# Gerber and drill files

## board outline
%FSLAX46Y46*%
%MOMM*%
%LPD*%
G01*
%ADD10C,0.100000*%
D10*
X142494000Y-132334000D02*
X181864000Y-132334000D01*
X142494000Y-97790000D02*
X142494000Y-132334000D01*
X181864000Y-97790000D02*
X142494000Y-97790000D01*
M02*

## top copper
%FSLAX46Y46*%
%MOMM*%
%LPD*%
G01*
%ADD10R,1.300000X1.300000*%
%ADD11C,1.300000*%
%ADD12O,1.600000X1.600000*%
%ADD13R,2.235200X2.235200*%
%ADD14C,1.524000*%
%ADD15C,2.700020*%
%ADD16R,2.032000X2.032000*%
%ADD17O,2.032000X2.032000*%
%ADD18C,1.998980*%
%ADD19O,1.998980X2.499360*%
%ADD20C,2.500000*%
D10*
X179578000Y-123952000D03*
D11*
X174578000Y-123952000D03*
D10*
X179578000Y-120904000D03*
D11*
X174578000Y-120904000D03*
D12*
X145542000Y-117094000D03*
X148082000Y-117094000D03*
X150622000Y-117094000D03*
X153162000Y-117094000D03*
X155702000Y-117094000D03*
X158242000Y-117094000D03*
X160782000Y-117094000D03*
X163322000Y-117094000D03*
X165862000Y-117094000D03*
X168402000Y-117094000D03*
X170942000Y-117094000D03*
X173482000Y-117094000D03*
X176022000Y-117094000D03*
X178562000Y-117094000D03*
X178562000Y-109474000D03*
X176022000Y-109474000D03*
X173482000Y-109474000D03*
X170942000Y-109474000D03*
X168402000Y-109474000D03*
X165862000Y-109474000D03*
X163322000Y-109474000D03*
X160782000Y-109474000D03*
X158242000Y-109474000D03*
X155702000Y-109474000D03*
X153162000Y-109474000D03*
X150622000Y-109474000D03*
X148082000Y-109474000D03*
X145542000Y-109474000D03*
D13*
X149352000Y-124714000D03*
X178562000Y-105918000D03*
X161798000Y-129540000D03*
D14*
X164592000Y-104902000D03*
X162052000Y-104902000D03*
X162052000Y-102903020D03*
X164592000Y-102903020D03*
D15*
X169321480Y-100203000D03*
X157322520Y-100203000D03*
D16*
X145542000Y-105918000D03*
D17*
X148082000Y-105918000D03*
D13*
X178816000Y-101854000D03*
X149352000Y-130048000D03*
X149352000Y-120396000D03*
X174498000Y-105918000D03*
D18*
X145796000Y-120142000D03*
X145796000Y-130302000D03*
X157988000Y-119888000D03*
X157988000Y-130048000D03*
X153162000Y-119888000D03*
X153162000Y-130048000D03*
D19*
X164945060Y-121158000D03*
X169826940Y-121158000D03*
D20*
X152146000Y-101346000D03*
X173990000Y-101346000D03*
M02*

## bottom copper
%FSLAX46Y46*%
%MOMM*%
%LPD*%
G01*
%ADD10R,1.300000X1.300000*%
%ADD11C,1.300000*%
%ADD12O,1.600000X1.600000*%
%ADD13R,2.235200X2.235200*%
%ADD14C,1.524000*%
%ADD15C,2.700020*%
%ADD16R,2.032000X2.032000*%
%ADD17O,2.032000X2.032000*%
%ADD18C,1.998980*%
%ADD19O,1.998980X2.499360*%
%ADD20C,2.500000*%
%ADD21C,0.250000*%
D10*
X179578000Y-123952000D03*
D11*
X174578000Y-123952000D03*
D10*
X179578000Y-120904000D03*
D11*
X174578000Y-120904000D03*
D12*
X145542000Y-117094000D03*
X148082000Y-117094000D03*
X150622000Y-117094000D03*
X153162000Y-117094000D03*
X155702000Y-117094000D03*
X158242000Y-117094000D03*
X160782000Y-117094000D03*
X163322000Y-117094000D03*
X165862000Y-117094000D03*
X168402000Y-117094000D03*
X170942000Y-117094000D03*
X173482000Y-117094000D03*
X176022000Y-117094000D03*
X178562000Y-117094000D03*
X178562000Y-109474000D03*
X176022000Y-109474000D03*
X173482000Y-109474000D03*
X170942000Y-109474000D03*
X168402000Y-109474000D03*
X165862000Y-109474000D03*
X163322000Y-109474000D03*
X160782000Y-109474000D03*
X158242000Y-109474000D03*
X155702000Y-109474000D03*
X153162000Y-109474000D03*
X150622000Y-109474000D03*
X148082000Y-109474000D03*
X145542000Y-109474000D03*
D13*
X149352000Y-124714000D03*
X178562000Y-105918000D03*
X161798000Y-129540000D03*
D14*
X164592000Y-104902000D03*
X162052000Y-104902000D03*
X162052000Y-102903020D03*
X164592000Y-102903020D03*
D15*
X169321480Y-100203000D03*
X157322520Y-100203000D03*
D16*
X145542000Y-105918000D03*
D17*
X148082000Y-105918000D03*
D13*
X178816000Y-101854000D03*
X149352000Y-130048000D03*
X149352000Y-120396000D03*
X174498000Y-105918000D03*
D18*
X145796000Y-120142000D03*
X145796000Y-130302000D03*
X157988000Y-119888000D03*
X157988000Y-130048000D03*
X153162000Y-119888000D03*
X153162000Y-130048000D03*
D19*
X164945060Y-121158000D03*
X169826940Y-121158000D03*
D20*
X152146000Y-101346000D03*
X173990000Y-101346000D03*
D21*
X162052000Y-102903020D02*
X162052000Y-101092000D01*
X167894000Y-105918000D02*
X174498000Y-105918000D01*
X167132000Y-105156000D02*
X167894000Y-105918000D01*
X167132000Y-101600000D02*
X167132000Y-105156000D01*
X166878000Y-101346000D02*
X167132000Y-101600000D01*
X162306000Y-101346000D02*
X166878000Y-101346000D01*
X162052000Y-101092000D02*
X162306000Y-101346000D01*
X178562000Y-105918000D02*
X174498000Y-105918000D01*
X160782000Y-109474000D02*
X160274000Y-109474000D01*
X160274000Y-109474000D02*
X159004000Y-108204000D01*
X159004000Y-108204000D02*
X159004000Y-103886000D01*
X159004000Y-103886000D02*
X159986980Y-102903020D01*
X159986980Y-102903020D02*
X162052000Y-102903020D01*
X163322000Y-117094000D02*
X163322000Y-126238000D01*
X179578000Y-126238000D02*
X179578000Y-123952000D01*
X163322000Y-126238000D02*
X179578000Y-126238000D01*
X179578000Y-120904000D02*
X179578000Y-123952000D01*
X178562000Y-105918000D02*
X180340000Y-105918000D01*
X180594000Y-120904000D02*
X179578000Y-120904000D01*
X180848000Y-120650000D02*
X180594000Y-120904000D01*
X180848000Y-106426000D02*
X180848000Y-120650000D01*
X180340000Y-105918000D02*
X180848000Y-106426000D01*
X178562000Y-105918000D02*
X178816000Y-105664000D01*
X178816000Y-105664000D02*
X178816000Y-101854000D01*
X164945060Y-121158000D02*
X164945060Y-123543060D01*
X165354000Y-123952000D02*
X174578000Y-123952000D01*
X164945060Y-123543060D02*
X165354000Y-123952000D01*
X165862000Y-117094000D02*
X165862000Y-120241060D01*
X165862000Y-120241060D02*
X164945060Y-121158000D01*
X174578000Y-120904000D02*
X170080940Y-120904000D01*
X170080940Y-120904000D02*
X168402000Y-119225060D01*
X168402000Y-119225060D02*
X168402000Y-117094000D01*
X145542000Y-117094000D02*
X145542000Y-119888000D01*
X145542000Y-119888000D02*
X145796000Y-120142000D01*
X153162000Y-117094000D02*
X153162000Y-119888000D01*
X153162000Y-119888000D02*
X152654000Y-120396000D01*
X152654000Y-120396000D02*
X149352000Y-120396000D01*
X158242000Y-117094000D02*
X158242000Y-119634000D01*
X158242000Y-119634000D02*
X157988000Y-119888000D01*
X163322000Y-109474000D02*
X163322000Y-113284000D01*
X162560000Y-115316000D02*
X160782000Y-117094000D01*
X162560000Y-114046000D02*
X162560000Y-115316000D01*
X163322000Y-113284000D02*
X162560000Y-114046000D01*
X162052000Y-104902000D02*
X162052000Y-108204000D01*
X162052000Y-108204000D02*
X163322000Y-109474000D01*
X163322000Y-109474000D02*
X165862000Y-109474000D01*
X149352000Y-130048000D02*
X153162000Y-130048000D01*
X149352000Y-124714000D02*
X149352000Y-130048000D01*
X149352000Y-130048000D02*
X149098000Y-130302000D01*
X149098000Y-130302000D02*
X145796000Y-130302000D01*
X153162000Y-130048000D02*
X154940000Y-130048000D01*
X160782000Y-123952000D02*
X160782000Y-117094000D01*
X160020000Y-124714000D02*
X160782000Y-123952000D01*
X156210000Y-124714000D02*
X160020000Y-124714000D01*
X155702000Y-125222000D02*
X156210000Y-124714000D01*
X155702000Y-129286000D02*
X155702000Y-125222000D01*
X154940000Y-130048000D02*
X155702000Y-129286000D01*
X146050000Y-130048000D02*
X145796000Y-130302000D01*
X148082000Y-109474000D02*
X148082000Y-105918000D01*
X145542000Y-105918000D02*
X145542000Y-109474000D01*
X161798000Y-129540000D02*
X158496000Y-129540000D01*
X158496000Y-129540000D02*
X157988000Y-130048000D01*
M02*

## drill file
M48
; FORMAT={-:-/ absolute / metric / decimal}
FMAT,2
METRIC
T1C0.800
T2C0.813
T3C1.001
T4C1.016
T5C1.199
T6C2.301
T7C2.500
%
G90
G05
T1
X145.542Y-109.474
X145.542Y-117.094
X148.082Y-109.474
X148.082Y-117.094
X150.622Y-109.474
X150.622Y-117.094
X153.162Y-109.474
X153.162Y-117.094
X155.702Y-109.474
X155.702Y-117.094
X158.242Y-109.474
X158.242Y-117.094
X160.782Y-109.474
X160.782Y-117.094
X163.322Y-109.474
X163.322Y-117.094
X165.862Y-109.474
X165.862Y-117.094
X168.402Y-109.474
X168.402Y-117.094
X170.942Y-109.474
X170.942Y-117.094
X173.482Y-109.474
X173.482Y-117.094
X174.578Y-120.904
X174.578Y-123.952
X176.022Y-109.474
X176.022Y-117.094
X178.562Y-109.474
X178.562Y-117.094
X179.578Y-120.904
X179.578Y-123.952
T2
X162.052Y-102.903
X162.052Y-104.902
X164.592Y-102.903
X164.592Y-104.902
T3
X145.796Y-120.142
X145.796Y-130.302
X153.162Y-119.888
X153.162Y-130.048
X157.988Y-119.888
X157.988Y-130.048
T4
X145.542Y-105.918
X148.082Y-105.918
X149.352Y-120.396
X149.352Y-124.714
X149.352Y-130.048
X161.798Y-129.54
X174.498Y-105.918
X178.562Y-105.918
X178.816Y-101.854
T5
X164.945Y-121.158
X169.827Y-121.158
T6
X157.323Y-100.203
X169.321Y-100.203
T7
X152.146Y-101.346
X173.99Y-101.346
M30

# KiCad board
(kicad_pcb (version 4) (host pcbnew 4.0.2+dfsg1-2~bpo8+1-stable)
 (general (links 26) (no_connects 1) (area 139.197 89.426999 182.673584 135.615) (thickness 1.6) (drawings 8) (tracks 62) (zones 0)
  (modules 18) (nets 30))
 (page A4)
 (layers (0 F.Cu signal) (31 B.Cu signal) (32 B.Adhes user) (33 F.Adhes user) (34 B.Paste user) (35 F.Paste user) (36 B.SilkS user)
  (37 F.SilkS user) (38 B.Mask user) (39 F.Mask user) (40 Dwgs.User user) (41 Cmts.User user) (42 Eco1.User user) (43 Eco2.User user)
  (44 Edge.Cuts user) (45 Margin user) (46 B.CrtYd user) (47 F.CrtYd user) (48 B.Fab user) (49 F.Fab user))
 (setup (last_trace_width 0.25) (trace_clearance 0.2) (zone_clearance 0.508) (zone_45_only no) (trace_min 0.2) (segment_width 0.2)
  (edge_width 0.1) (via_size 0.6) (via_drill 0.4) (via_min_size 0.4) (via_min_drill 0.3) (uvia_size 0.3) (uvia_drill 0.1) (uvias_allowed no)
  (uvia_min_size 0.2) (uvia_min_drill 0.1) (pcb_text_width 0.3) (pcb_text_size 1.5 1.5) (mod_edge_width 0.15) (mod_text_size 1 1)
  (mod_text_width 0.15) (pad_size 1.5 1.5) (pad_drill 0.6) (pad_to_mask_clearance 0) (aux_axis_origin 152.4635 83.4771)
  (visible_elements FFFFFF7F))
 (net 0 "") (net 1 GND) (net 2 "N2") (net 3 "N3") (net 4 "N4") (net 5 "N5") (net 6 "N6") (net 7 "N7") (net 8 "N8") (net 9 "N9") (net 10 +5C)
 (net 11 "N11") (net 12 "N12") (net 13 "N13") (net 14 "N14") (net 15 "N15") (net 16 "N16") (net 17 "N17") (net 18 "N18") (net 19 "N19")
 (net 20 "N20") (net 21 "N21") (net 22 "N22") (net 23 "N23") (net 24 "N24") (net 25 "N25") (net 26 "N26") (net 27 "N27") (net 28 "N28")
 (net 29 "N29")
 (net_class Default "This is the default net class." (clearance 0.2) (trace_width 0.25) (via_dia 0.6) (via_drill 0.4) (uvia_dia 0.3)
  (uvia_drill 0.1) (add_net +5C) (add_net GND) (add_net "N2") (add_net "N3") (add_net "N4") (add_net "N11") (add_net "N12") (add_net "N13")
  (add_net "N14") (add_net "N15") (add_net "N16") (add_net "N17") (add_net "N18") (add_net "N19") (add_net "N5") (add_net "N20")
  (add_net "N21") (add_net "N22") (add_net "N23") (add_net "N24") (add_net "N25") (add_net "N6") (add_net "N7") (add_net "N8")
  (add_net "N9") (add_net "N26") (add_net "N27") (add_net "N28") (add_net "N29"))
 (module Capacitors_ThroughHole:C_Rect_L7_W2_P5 (layer F.Cu) (at 179.578 123.952 180)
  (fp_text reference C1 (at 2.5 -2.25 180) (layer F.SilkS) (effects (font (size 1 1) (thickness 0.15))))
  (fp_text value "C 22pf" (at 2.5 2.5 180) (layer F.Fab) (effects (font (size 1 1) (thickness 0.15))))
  (pad 1 thru_hole rect (at 0 0 180) (size 1.3 1.3) (drill 0.8) (layers *.Cu *.Mask F.SilkS) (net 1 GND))
  (pad 2 thru_hole circle (at 5 0 180) (size 1.3 1.3) (drill 0.8) (layers *.Cu *.Mask F.SilkS) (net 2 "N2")))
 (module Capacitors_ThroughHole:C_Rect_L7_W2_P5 (layer F.Cu) (at 179.578 120.904 180)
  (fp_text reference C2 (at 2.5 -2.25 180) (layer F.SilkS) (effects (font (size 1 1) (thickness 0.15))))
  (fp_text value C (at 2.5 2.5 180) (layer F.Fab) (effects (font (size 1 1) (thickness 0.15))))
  (pad 1 thru_hole rect (at 0 0 180) (size 1.3 1.3) (drill 0.8) (layers *.Cu *.Mask F.SilkS) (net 1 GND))
  (pad 2 thru_hole circle (at 5 0 180) (size 1.3 1.3) (drill 0.8) (layers *.Cu *.Mask F.SilkS) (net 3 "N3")))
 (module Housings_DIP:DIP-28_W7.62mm (layer F.Cu) (at 145.542 117.094 90)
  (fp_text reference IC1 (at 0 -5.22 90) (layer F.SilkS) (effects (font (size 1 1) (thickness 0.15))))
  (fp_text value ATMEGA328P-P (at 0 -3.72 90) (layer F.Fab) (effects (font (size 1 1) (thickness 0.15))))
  (pad 1 thru_hole oval (at 0 0 90) (size 1.6 1.6) (drill 0.8) (layers *.Cu *.Mask F.SilkS) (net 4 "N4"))
  (pad 2 thru_hole oval (at 0 2.54 90) (size 1.6 1.6) (drill 0.8) (layers *.Cu *.Mask F.SilkS) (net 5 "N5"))
  (pad 3 thru_hole oval (at 0 5.08 90) (size 1.6 1.6) (drill 0.8) (layers *.Cu *.Mask F.SilkS) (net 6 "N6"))
  (pad 4 thru_hole oval (at 0 7.62 90) (size 1.6 1.6) (drill 0.8) (layers *.Cu *.Mask F.SilkS) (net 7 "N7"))
  (pad 5 thru_hole oval (at 0 10.16 90) (size 1.6 1.6) (drill 0.8) (layers *.Cu *.Mask F.SilkS) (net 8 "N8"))
  (pad 6 thru_hole oval (at 0 12.7 90) (size 1.6 1.6) (drill 0.8) (layers *.Cu *.Mask F.SilkS) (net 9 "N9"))
  (pad 7 thru_hole oval (at 0 15.24 90) (size 1.6 1.6) (drill 0.8) (layers *.Cu *.Mask F.SilkS) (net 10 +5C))
  (pad 8 thru_hole oval (at 0 17.78 90) (size 1.6 1.6) (drill 0.8) (layers *.Cu *.Mask F.SilkS) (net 1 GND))
  (pad 9 thru_hole oval (at 0 20.32 90) (size 1.6 1.6) (drill 0.8) (layers *.Cu *.Mask F.SilkS) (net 2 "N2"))
  (pad 10 thru_hole oval (at 0 22.86 90) (size 1.6 1.6) (drill 0.8) (layers *.Cu *.Mask F.SilkS) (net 3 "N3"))
  (pad 11 thru_hole oval (at 0 25.4 90) (size 1.6 1.6) (drill 0.8) (layers *.Cu *.Mask F.SilkS) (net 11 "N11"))
  (pad 12 thru_hole oval (at 0 27.94 90) (size 1.6 1.6) (drill 0.8) (layers *.Cu *.Mask F.SilkS) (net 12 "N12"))
  (pad 13 thru_hole oval (at 0 30.48 90) (size 1.6 1.6) (drill 0.8) (layers *.Cu *.Mask F.SilkS) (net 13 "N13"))
  (pad 14 thru_hole oval (at 0 33.02 90) (size 1.6 1.6) (drill 0.8) (layers *.Cu *.Mask F.SilkS) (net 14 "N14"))
  (pad 15 thru_hole oval (at 7.62 33.02 90) (size 1.6 1.6) (drill 0.8) (layers *.Cu *.Mask F.SilkS) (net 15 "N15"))
  (pad 16 thru_hole oval (at 7.62 30.48 90) (size 1.6 1.6) (drill 0.8) (layers *.Cu *.Mask F.SilkS) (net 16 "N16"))
  (pad 17 thru_hole oval (at 7.62 27.94 90) (size 1.6 1.6) (drill 0.8) (layers *.Cu *.Mask F.SilkS) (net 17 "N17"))
  (pad 18 thru_hole oval (at 7.62 25.4 90) (size 1.6 1.6) (drill 0.8) (layers *.Cu *.Mask F.SilkS) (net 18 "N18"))
  (pad 19 thru_hole oval (at 7.62 22.86 90) (size 1.6 1.6) (drill 0.8) (layers *.Cu *.Mask F.SilkS) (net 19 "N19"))
  (pad 20 thru_hole oval (at 7.62 20.32 90) (size 1.6 1.6) (drill 0.8) (layers *.Cu *.Mask F.SilkS) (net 10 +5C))
  (pad 21 thru_hole oval (at 7.62 17.78 90) (size 1.6 1.6) (drill 0.8) (layers *.Cu *.Mask F.SilkS) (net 10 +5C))
  (pad 22 thru_hole oval (at 7.62 15.24 90) (size 1.6 1.6) (drill 0.8) (layers *.Cu *.Mask F.SilkS) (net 1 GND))
  (pad 23 thru_hole oval (at 7.62 12.7 90) (size 1.6 1.6) (drill 0.8) (layers *.Cu *.Mask F.SilkS) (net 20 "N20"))
  (pad 24 thru_hole oval (at 7.62 10.16 90) (size 1.6 1.6) (drill 0.8) (layers *.Cu *.Mask F.SilkS) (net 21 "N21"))
  (pad 25 thru_hole oval (at 7.62 7.62 90) (size 1.6 1.6) (drill 0.8) (layers *.Cu *.Mask F.SilkS) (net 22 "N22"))
  (pad 26 thru_hole oval (at 7.62 5.08 90) (size 1.6 1.6) (drill 0.8) (layers *.Cu *.Mask F.SilkS) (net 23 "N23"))
  (pad 27 thru_hole oval (at 7.62 2.54 90) (size 1.6 1.6) (drill 0.8) (layers *.Cu *.Mask F.SilkS) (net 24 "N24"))
  (pad 28 thru_hole oval (at 7.62 0 90) (size 1.6 1.6) (drill 0.8) (layers *.Cu *.Mask F.SilkS) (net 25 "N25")))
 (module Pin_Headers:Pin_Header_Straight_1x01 (layer F.Cu) (at 149.352 124.714)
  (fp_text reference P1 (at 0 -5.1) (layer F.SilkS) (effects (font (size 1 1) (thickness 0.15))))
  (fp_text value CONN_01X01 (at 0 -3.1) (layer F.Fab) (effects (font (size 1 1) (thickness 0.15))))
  (pad 1 thru_hole rect (at 0 0) (size 2.2352 2.2352) (drill 1.016) (layers *.Cu *.Mask F.SilkS) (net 10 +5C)))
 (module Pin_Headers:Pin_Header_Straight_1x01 (layer F.Cu) (at 178.562 105.918 90)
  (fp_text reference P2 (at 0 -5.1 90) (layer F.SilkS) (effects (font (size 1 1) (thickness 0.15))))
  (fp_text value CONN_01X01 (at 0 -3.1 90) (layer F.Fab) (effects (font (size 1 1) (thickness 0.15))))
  (pad 1 thru_hole rect (at 0 0 90) (size 2.2352 2.2352) (drill 1.016) (layers *.Cu *.Mask F.SilkS) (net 1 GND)))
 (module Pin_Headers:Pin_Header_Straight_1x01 (layer F.Cu) (at 161.798 129.54 180)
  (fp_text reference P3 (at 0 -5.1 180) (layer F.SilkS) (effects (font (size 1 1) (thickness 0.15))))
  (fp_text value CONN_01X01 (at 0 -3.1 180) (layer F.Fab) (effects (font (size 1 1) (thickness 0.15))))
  (pad 1 thru_hole rect (at 0 0 180) (size 2.2352 2.2352) (drill 1.016) (layers *.Cu *.Mask F.SilkS) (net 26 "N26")))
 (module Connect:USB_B (layer F.Cu) (at 162.052 104.902 90)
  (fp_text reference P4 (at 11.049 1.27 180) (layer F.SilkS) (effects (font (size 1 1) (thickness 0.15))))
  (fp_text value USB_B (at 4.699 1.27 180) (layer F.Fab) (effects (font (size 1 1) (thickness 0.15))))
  (pad 2 thru_hole circle (at 0 2.54) (size 1.524 1.524) (drill 0.8128) (layers *.Cu *.Mask F.SilkS) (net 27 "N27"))
  (pad 1 thru_hole circle (at 0 0) (size 1.524 1.524) (drill 0.8128) (layers *.Cu *.Mask F.SilkS) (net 10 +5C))
  (pad 4 thru_hole circle (at 1.99898 0) (size 1.524 1.524) (drill 0.8128) (layers *.Cu *.Mask F.SilkS) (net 1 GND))
  (pad 3 thru_hole circle (at 1.99898 2.54) (size 1.524 1.524) (drill 0.8128) (layers *.Cu *.Mask F.SilkS) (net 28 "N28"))
  (pad 5 thru_hole circle (at 4.699 7.26948) (size 2.70002 2.70002) (drill 2.30124) (layers *.Cu *.Mask F.SilkS) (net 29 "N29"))
  (pad 5 thru_hole circle (at 4.699 -4.72948) (size 2.70002 2.70002) (drill 2.30124) (layers *.Cu *.Mask F.SilkS) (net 29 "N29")))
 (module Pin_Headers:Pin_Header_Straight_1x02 (layer F.Cu) (at 145.542 105.918 90)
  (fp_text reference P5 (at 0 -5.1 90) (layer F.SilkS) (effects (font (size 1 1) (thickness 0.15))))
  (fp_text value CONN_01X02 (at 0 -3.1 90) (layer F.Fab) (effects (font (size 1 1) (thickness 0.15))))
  (pad 1 thru_hole rect (at 0 0 90) (size 2.032 2.032) (drill 1.016) (layers *.Cu *.Mask F.SilkS) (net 25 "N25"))
  (pad 2 thru_hole oval (at 0 2.54 90) (size 2.032 2.032) (drill 1.016) (layers *.Cu *.Mask F.SilkS) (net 24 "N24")))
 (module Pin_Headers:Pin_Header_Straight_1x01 (layer F.Cu) (at 178.816 101.854 90)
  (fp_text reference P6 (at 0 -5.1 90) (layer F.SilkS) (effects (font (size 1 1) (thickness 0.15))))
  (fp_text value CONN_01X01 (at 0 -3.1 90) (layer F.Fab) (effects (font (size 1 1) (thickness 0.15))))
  (pad 1 thru_hole rect (at 0 0 90) (size 2.2352 2.2352) (drill 1.016) (layers *.Cu *.Mask F.SilkS) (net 1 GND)))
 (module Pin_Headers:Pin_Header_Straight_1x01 (layer F.Cu) (at 149.352 130.048)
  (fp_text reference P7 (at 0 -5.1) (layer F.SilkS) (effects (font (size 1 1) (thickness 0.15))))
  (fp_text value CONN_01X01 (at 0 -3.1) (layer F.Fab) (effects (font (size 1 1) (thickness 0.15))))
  (pad 1 thru_hole rect (at 0 0) (size 2.2352 2.2352) (drill 1.016) (layers *.Cu *.Mask F.SilkS) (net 10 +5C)))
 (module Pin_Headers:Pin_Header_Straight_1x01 (layer F.Cu) (at 149.352 120.396 90)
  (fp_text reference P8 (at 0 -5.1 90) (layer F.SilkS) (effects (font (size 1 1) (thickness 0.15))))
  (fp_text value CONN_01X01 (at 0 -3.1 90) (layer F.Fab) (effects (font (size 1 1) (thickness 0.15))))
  (pad 1 thru_hole rect (at 0 0 90) (size 2.2352 2.2352) (drill 1.016) (layers *.Cu *.Mask F.SilkS) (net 7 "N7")))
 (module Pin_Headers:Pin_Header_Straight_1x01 (layer F.Cu) (at 174.498 105.918 90)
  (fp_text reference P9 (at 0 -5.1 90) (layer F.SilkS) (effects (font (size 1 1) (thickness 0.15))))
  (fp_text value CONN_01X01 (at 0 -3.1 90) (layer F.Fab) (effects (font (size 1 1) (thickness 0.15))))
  (pad 1 thru_hole rect (at 0 0 90) (size 2.2352 2.2352) (drill 1.016) (layers *.Cu *.Mask F.SilkS) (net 1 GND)))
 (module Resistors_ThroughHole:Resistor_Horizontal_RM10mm (layer F.Cu) (at 145.796 120.142 270)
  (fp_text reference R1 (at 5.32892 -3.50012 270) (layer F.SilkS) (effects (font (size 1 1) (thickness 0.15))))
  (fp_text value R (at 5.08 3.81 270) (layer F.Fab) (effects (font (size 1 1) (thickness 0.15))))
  (pad 1 thru_hole circle (at 0 0 270) (size 1.99898 1.99898) (drill 1.00076) (layers *.Cu *.SilkS *.Mask) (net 4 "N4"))
  (pad 2 thru_hole circle (at 10.16 0 270) (size 1.99898 1.99898) (drill 1.00076) (layers *.Cu *.SilkS *.Mask) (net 10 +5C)))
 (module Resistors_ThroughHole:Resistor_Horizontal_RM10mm (layer F.Cu) (at 157.988 119.888 270)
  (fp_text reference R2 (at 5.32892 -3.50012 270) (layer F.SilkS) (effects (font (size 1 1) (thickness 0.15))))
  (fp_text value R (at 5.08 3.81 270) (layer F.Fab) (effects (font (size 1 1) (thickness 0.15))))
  (pad 1 thru_hole circle (at 0 0 270) (size 1.99898 1.99898) (drill 1.00076) (layers *.Cu *.SilkS *.Mask) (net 9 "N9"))
  (pad 2 thru_hole circle (at 10.16 0 270) (size 1.99898 1.99898) (drill 1.00076) (layers *.Cu *.SilkS *.Mask) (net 26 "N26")))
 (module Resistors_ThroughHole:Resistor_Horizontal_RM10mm (layer F.Cu) (at 153.162 119.888 270)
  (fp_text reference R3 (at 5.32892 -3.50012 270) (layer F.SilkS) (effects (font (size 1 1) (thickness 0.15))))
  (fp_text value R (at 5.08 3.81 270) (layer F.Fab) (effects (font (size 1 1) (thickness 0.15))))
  (pad 1 thru_hole circle (at 0 0 270) (size 1.99898 1.99898) (drill 1.00076) (layers *.Cu *.SilkS *.Mask) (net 7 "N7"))
  (pad 2 thru_hole circle (at 10.16 0 270) (size 1.99898 1.99898) (drill 1.00076) (layers *.Cu *.SilkS *.Mask) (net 10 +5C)))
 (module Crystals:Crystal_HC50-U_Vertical (layer F.Cu) (at 167.386 121.158)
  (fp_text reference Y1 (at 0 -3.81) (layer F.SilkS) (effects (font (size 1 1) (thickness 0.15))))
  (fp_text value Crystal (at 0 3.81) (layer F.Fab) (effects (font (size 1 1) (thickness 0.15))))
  (pad 1 thru_hole oval (at -2.44094 0) (size 1.99898 2.49936) (drill 1.19888) (layers *.Cu *.Mask F.SilkS) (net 2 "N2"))
  (pad 2 thru_hole oval (at 2.44094 0) (size 1.99898 2.49936) (drill 1.19888) (layers *.Cu *.Mask F.SilkS) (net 3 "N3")))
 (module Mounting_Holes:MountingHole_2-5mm (layer F.Cu) (at 152.146 101.346)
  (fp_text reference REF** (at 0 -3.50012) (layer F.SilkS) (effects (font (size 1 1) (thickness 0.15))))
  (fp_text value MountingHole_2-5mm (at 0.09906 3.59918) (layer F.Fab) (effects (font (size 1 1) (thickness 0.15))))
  (pad 1 thru_hole circle (at 0 0) (size 2.5 2.5) (drill 2.5) (layers)))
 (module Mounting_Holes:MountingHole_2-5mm (layer F.Cu) (at 173.99 101.346)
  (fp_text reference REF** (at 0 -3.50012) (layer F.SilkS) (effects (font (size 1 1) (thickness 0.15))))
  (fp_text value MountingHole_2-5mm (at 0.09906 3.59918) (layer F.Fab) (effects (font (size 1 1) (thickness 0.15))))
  (pad 1 thru_hole circle (at 0 0) (size 2.5 2.5) (drill 2.5) (layers)))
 (gr_line (start 142.494 132.334) (end 181.864 132.334) (angle 90) (layer Edge.Cuts) (width 0.1))
 (gr_line (start 142.494 97.79) (end 142.494 132.334) (angle 90) (layer Edge.Cuts) (width 0.1))
 (gr_line (start 181.864 97.79) (end 142.494 97.79) (angle 90) (layer Edge.Cuts) (width 0.1))
 (segment (start 162.052 102.90302) (end 162.052 101.092) (width 0.25) (layer B.Cu) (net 1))
 (segment (start 167.894 105.918) (end 174.498 105.918) (width 0.25) (layer B.Cu) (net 1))
 (segment (start 167.132 105.156) (end 167.894 105.918) (width 0.25) (layer B.Cu) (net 1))
 (segment (start 167.132 101.6) (end 167.132 105.156) (width 0.25) (layer B.Cu) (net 1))
 (segment (start 166.878 101.346) (end 167.132 101.6) (width 0.25) (layer B.Cu) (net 1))
 (segment (start 162.306 101.346) (end 166.878 101.346) (width 0.25) (layer B.Cu) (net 1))
 (segment (start 162.052 101.092) (end 162.306 101.346) (width 0.25) (layer B.Cu) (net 1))
 (segment (start 178.562 105.918) (end 174.498 105.918) (width 0.25) (layer B.Cu) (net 1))
 (segment (start 160.782 109.474) (end 160.274 109.474) (width 0.25) (layer B.Cu) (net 1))
 (segment (start 160.274 109.474) (end 159.004 108.204) (width 0.25) (layer B.Cu) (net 1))
 (segment (start 159.004 108.204) (end 159.004 103.886) (width 0.25) (layer B.Cu) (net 1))
 (segment (start 159.004 103.886) (end 159.98698 102.90302) (width 0.25) (layer B.Cu) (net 1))
 (segment (start 159.98698 102.90302) (end 162.052 102.90302) (width 0.25) (layer B.Cu) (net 1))
 (segment (start 163.322 117.094) (end 163.322 126.238) (width 0.25) (layer B.Cu) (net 1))
 (segment (start 179.578 126.238) (end 179.578 123.952) (width 0.25) (layer B.Cu) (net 1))
 (segment (start 163.322 126.238) (end 179.578 126.238) (width 0.25) (layer B.Cu) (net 1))
 (segment (start 179.578 120.904) (end 179.578 123.952) (width 0.25) (layer B.Cu) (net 1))
 (segment (start 178.562 105.918) (end 180.34 105.918) (width 0.25) (layer B.Cu) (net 1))
 (segment (start 180.594 120.904) (end 179.578 120.904) (width 0.25) (layer B.Cu) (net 1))
 (segment (start 180.848 120.65) (end 180.594 120.904) (width 0.25) (layer B.Cu) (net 1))
 (segment (start 180.848 106.426) (end 180.848 120.65) (width 0.25) (layer B.Cu) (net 1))
 (segment (start 180.34 105.918) (end 180.848 106.426) (width 0.25) (layer B.Cu) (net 1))
 (segment (start 178.562 105.918) (end 178.816 105.664) (width 0.25) (layer B.Cu) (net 1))
 (segment (start 178.816 105.664) (end 178.816 101.854) (width 0.25) (layer B.Cu) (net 1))
 (segment (start 164.94506 121.158) (end 164.94506 123.54306) (width 0.25) (layer B.Cu) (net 2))
 (segment (start 165.354 123.952) (end 174.578 123.952) (width 0.25) (layer B.Cu) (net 2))
 (segment (start 164.94506 123.54306) (end 165.354 123.952) (width 0.25) (layer B.Cu) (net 2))
 (segment (start 165.862 117.094) (end 165.862 120.24106) (width 0.25) (layer B.Cu) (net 2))
 (segment (start 165.862 120.24106) (end 164.94506 121.158) (width 0.25) (layer B.Cu) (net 2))
 (segment (start 174.578 120.904) (end 170.08094 120.904) (width 0.25) (layer B.Cu) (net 3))
 (segment (start 170.08094 120.904) (end 168.402 119.22506) (width 0.25) (layer B.Cu) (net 3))
 (segment (start 168.402 119.22506) (end 168.402 117.094) (width 0.25) (layer B.Cu) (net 3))
 (segment (start 145.542 117.094) (end 145.542 119.888) (width 0.25) (layer B.Cu) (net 4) (status C00000))
 (segment (start 145.542 119.888) (end 145.796 120.142) (width 0.25) (layer B.Cu) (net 4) (status C00000))
 (segment (start 153.162 117.094) (end 153.162 119.888) (width 0.25) (layer B.Cu) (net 7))
 (segment (start 153.162 119.888) (end 152.654 120.396) (width 0.25) (layer B.Cu) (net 7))
 (segment (start 152.654 120.396) (end 149.352 120.396) (width 0.25) (layer B.Cu) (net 7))
 (segment (start 158.242 117.094) (end 158.242 119.634) (width 0.25) (layer B.Cu) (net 9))
 (segment (start 158.242 119.634) (end 157.988 119.888) (width 0.25) (layer B.Cu) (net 9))
 (segment (start 163.322 109.474) (end 163.322 113.284) (width 0.25) (layer B.Cu) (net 10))
 (segment (start 162.56 115.316) (end 160.782 117.094) (width 0.25) (layer B.Cu) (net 10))
 (segment (start 162.56 114.046) (end 162.56 115.316) (width 0.25) (layer B.Cu) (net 10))
 (segment (start 163.322 113.284) (end 162.56 114.046) (width 0.25) (layer B.Cu) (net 10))
 (segment (start 162.052 104.902) (end 162.052 108.204) (width 0.25) (layer B.Cu) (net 10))
 (segment (start 162.052 108.204) (end 163.322 109.474) (width 0.25) (layer B.Cu) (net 10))
 (segment (start 163.322 109.474) (end 165.862 109.474) (width 0.25) (layer B.Cu) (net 10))
 (segment (start 149.352 130.048) (end 153.162 130.048) (width 0.25) (layer B.Cu) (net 10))
 (segment (start 149.352 124.714) (end 149.352 130.048) (width 0.25) (layer B.Cu) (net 10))
 (segment (start 149.352 130.048) (end 149.098 130.302) (width 0.25) (layer B.Cu) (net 10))
 (segment (start 149.098 130.302) (end 145.796 130.302) (width 0.25) (layer B.Cu) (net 10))
 (segment (start 153.162 130.048) (end 154.94 130.048) (width 0.25) (layer B.Cu) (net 10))
 (segment (start 160.782 123.952) (end 160.782 117.094) (width 0.25) (layer B.Cu) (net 10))
 (segment (start 160.02 124.714) (end 160.782 123.952) (width 0.25) (layer B.Cu) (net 10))
 (segment (start 156.21 124.714) (end 160.02 124.714) (width 0.25) (layer B.Cu) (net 10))
 (segment (start 155.702 125.222) (end 156.21 124.714) (width 0.25) (layer B.Cu) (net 10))
 (segment (start 155.702 129.286) (end 155.702 125.222) (width 0.25) (layer B.Cu) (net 10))
 (segment (start 154.94 130.048) (end 155.702 129.286) (width 0.25) (layer B.Cu) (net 10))
 (segment (start 146.05 130.048) (end 145.796 130.302) (width 0.25) (layer B.Cu) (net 10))
 (segment (start 148.082 109.474) (end 148.082 105.918) (width 0.25) (layer B.Cu) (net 24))
 (segment (start 145.542 105.918) (end 145.542 109.474) (width 0.25) (layer B.Cu) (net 25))
 (segment (start 161.798 129.54) (end 158.496 129.54) (width 0.25) (layer B.Cu) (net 26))
 (segment (start 158.496 129.54) (end 157.988 130.048) (width 0.25) (layer B.Cu) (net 26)))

